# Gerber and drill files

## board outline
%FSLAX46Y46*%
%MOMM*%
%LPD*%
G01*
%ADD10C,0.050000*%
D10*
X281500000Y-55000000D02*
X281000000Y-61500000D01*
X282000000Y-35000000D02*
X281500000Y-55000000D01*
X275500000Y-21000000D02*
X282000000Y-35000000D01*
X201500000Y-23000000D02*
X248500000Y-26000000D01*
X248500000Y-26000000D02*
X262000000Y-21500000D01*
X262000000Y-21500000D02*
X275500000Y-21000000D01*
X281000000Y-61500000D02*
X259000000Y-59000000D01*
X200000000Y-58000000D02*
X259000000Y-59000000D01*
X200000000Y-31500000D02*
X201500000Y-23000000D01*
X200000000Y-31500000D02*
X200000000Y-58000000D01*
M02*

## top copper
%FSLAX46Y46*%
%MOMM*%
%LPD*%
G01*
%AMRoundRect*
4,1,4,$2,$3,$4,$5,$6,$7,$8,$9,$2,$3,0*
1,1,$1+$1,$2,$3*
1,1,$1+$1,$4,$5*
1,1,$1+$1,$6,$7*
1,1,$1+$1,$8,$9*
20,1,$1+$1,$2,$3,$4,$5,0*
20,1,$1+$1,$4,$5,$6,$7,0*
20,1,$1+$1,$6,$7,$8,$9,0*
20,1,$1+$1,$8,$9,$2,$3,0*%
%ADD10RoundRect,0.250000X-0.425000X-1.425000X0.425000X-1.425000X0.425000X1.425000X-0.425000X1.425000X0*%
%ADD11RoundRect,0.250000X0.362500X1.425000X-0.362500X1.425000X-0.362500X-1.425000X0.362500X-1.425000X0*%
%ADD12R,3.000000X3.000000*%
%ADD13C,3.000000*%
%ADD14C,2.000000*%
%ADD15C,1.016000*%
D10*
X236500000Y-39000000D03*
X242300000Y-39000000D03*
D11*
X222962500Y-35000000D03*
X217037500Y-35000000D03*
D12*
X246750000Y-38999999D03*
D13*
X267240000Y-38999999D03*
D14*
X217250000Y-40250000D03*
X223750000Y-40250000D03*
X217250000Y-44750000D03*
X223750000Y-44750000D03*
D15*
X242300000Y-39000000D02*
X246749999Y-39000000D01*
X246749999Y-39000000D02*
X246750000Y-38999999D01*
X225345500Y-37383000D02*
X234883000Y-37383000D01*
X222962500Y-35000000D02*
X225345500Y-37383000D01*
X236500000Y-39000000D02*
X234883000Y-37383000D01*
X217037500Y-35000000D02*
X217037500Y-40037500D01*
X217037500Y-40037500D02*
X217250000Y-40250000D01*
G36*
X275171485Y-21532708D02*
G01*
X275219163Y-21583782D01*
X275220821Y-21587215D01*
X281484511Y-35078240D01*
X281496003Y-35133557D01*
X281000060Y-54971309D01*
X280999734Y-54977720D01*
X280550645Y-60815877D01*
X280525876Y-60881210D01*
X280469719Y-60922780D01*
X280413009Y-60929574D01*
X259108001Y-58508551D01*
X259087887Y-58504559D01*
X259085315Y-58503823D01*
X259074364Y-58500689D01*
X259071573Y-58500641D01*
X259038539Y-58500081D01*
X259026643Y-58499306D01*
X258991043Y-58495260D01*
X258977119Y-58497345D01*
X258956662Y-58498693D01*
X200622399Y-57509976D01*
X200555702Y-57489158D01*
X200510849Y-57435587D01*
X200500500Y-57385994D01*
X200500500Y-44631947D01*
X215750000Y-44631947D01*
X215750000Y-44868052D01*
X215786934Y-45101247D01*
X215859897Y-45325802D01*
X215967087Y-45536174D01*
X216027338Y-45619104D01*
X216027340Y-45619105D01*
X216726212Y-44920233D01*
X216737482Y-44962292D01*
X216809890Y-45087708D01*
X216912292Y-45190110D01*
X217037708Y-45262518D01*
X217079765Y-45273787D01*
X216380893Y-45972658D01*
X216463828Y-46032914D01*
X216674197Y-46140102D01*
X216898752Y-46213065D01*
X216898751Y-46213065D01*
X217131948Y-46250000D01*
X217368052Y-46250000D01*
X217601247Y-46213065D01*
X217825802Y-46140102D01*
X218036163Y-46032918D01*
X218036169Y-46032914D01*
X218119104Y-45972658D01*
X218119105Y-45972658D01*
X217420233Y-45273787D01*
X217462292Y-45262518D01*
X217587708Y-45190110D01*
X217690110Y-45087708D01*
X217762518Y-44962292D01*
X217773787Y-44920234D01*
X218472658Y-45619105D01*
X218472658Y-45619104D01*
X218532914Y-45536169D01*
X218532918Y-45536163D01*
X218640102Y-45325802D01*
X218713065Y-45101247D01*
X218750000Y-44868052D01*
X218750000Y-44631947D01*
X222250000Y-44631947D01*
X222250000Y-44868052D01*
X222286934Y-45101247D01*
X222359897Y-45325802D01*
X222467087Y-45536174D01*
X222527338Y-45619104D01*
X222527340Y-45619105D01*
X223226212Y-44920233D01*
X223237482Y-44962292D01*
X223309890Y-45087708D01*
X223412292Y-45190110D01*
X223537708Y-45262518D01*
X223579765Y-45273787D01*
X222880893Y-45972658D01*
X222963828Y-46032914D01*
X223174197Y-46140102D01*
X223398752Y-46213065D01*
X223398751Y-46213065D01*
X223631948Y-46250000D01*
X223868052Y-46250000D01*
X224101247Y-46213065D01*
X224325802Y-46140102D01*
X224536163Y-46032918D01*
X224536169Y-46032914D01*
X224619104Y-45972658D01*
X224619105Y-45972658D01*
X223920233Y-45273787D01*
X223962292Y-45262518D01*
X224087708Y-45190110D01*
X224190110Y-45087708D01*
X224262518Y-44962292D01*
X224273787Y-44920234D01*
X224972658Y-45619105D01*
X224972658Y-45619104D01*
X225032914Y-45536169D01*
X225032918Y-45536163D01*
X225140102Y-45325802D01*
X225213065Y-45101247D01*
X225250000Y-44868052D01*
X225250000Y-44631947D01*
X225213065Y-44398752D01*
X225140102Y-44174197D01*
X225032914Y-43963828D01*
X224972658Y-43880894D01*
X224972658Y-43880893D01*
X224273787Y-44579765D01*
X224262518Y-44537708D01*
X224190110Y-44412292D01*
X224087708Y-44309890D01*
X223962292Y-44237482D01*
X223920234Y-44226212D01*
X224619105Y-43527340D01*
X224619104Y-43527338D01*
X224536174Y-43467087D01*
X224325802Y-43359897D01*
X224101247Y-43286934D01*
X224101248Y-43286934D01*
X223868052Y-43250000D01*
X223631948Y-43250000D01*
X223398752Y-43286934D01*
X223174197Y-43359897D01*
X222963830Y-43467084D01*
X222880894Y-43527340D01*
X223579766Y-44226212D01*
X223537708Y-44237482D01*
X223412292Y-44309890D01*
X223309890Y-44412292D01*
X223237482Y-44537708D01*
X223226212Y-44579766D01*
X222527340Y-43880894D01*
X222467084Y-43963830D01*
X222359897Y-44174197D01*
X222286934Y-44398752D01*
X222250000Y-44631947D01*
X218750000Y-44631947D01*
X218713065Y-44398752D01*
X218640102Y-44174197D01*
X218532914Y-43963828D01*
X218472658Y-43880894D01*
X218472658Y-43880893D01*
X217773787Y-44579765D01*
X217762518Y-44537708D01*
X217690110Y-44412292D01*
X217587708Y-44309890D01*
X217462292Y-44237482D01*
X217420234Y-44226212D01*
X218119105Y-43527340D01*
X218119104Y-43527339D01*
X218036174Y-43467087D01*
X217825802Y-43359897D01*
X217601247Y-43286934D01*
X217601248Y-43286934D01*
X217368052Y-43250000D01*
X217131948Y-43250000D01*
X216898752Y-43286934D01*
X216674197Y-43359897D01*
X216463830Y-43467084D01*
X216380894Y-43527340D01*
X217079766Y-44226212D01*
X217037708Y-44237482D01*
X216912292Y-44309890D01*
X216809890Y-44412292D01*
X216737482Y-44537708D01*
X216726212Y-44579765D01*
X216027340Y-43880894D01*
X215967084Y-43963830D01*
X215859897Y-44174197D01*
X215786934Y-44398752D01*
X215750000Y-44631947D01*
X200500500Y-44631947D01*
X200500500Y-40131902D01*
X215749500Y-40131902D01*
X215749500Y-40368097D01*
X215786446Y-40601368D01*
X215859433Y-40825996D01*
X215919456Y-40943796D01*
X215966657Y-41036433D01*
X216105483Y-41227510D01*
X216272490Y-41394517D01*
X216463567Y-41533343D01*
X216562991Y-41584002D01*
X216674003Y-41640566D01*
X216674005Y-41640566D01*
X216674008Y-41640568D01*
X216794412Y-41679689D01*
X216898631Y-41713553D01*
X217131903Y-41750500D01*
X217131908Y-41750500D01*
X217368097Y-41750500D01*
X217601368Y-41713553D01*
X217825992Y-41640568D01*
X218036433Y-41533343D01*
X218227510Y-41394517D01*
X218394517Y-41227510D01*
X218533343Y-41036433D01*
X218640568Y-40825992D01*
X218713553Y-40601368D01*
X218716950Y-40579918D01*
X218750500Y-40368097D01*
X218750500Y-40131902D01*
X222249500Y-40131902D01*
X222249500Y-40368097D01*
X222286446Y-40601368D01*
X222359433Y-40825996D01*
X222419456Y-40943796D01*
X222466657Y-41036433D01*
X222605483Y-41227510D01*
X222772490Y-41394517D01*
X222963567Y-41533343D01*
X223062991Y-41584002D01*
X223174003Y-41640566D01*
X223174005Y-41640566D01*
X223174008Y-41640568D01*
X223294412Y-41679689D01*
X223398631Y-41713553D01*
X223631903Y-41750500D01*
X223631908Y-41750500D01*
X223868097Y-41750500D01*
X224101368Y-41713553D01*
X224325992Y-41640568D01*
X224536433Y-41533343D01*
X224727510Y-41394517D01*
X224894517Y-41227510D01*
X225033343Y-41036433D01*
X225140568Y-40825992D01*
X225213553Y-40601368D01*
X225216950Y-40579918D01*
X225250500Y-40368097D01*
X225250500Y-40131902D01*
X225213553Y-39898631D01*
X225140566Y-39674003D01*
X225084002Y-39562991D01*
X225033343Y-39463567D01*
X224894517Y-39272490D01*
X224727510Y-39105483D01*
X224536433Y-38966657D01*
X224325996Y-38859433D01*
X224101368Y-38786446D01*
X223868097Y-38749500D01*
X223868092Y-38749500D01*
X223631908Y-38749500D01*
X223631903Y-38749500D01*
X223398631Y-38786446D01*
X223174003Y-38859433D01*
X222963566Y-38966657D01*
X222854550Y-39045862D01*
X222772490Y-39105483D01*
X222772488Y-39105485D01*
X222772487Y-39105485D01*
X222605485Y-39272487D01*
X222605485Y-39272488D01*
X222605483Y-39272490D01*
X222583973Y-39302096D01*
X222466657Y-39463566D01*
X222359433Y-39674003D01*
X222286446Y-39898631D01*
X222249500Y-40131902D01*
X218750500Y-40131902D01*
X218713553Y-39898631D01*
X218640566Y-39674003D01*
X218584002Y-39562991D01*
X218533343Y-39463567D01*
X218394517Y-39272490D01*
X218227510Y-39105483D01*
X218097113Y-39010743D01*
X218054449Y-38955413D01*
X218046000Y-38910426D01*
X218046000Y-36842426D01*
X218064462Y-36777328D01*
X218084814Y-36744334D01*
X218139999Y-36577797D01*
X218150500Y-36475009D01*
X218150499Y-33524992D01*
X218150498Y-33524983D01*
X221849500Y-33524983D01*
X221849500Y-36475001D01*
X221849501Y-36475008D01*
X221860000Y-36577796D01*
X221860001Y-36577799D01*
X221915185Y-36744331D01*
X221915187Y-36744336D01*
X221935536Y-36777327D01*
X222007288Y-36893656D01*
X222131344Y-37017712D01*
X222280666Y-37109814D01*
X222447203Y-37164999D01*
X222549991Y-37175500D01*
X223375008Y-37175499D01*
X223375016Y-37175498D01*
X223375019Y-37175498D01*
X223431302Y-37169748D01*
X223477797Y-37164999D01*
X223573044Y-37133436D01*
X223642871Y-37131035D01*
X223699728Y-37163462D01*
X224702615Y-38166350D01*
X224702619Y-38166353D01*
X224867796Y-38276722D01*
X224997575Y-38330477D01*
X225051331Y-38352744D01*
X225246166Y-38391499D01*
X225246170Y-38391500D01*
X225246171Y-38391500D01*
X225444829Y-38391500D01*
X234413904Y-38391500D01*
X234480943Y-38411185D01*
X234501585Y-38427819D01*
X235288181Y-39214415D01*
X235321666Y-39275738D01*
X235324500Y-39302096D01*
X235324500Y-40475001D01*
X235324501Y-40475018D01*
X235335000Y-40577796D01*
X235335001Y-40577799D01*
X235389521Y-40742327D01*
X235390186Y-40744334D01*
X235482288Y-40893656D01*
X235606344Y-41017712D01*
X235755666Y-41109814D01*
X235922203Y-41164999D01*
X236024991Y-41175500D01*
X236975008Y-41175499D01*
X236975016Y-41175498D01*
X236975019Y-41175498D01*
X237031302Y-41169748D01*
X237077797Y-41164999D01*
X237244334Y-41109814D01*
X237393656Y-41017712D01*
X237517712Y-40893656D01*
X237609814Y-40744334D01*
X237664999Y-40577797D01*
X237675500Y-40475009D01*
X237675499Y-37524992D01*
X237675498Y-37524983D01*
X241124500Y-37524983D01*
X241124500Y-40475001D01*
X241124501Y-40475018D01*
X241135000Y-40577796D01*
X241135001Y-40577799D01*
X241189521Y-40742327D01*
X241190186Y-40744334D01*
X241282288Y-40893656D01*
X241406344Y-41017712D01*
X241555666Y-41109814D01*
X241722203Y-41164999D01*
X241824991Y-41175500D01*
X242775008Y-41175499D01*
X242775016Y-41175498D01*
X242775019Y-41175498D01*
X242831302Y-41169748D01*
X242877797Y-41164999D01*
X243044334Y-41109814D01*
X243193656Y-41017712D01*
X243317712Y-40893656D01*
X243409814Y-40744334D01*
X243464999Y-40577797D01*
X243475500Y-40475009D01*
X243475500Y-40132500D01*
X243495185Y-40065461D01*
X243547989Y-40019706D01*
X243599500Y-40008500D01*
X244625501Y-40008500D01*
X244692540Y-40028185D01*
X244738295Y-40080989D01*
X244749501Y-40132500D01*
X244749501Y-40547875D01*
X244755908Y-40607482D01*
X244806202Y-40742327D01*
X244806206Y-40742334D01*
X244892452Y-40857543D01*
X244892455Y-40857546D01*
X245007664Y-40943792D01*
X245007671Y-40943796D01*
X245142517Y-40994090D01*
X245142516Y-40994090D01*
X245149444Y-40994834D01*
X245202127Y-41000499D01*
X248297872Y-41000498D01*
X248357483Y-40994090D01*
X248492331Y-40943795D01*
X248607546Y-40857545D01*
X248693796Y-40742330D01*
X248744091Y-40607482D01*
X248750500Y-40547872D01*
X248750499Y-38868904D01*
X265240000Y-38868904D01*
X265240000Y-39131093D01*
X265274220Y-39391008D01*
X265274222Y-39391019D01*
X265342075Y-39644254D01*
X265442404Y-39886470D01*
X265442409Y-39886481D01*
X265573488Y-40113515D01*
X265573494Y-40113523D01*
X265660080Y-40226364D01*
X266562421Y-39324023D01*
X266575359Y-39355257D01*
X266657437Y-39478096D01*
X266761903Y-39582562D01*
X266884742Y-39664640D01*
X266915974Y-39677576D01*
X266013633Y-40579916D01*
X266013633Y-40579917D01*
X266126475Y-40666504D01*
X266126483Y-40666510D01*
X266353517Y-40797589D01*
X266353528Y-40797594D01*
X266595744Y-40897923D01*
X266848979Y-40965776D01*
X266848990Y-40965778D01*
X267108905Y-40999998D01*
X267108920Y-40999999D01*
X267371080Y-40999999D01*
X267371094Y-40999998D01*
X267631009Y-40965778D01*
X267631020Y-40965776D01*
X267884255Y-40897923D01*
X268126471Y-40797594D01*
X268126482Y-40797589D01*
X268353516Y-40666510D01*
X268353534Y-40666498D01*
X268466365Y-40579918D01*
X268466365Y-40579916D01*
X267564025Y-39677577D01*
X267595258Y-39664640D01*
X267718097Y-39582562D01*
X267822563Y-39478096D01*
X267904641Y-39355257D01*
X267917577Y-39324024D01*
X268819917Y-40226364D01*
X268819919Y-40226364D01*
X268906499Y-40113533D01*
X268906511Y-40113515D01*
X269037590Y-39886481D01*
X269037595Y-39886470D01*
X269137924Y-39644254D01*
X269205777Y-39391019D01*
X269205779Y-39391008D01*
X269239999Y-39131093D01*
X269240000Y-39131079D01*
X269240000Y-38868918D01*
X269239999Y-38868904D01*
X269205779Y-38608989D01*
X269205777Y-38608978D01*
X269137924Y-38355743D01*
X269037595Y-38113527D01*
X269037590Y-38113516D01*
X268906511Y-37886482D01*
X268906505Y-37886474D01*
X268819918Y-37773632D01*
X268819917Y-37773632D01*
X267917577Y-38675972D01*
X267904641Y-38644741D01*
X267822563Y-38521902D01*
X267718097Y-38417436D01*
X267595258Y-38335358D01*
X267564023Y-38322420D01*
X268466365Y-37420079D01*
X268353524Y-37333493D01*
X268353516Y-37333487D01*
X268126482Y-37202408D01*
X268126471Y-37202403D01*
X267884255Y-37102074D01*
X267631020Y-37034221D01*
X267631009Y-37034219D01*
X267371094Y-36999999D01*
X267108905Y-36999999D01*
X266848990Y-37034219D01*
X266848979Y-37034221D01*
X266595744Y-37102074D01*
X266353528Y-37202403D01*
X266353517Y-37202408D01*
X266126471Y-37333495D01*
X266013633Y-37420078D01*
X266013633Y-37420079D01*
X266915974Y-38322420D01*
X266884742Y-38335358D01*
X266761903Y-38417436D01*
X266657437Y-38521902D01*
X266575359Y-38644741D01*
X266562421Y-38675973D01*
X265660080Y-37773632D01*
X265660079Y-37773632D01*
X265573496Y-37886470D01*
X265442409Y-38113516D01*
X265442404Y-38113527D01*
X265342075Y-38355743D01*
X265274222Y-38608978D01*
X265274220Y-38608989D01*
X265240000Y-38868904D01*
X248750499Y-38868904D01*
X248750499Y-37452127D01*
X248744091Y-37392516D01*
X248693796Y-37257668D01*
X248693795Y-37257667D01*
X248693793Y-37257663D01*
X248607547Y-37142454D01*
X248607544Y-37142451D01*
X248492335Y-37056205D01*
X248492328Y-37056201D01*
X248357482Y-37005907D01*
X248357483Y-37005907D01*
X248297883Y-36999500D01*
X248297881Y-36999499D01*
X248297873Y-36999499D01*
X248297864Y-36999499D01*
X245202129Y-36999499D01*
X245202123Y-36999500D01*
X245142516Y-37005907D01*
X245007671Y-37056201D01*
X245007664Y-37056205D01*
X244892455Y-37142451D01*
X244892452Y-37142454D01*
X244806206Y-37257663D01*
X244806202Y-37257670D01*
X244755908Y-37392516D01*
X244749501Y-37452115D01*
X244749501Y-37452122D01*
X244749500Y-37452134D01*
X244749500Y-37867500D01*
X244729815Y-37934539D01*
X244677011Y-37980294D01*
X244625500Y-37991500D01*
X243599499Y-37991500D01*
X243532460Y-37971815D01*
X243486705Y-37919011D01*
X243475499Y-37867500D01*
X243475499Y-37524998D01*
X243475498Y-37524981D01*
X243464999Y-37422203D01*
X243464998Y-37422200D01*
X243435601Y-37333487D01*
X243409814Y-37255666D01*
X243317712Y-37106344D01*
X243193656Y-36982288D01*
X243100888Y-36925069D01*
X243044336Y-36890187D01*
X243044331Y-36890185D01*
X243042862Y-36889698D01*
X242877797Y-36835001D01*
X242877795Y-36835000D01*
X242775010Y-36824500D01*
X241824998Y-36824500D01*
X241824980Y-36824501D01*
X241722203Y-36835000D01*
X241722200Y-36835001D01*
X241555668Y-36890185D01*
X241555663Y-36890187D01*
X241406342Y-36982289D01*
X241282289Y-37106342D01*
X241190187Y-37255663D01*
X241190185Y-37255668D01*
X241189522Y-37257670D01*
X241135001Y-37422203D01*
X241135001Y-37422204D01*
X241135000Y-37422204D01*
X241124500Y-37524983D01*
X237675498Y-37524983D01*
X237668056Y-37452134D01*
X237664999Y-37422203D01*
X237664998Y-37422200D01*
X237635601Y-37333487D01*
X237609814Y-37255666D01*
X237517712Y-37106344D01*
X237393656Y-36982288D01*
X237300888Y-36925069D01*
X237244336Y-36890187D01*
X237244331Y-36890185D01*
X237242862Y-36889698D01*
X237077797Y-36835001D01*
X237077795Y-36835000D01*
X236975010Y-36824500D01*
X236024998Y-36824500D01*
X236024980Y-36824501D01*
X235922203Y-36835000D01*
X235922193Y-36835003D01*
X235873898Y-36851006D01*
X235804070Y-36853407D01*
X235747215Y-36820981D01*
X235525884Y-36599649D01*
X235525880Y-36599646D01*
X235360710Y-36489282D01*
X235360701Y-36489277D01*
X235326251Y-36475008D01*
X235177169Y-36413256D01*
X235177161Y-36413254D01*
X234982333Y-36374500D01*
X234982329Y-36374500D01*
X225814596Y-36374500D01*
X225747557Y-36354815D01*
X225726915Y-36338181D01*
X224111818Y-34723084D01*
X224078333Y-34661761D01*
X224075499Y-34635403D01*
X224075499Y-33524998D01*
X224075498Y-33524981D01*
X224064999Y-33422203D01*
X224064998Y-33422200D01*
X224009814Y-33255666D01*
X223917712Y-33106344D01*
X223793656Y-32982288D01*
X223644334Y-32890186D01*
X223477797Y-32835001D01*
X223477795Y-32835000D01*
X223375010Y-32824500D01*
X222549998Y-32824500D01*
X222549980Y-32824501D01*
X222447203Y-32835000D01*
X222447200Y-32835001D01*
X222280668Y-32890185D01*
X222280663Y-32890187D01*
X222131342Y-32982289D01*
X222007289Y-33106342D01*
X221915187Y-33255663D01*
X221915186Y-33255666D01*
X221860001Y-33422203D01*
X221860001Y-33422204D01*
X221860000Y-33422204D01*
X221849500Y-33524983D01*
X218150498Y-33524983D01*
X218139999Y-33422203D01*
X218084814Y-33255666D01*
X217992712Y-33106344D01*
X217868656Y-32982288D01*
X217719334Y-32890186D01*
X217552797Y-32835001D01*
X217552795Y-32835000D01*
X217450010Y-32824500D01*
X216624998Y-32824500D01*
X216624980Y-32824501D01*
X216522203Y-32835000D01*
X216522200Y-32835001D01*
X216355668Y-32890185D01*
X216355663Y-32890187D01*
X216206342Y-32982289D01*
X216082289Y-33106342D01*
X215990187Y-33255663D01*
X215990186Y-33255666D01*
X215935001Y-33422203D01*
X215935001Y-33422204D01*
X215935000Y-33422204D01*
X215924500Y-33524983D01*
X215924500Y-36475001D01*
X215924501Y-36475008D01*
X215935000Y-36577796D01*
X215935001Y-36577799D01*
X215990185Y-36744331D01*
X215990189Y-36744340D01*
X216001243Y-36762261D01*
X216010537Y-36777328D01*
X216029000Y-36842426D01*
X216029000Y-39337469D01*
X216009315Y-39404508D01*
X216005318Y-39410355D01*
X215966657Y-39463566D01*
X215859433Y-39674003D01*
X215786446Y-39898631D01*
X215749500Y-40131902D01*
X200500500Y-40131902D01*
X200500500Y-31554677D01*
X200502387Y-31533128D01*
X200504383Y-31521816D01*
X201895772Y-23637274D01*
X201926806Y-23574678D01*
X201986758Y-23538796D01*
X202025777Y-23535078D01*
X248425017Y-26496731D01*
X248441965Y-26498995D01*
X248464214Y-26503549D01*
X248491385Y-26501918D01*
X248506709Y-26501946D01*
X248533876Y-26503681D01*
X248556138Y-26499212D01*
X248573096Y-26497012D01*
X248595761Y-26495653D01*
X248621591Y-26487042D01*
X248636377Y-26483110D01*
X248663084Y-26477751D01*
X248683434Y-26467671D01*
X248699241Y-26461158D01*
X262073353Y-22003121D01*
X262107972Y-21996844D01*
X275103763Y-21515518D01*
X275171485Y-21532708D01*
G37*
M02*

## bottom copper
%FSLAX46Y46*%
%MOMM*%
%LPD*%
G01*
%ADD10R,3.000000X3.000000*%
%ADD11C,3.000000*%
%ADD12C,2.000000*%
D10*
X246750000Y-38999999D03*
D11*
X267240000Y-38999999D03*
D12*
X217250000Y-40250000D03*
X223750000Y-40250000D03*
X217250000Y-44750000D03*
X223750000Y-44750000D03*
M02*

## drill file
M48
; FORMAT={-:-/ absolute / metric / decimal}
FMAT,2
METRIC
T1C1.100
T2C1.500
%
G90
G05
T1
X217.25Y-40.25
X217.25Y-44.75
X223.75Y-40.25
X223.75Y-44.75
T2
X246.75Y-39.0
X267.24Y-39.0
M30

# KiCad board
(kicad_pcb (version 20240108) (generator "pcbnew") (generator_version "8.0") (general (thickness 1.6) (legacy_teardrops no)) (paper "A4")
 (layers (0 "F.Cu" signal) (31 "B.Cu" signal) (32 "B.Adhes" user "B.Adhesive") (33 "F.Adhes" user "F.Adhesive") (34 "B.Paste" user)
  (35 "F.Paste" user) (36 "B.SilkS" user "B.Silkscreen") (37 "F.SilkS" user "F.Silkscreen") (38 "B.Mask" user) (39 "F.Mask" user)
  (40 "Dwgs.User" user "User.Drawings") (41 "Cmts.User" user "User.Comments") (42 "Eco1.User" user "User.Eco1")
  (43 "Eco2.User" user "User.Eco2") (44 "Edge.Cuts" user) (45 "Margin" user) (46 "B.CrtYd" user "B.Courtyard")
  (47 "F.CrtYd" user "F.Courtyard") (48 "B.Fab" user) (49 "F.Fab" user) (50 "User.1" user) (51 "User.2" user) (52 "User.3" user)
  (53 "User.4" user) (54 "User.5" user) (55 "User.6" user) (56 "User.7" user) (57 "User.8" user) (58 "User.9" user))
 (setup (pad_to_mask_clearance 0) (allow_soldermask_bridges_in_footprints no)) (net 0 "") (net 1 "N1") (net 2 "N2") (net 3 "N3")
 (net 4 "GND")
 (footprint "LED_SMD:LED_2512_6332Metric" (layer "F.Cu") (at 239.4 39)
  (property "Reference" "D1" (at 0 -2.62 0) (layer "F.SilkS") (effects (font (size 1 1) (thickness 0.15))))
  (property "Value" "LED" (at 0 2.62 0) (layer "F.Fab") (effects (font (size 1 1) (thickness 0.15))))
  (pad "1" smd roundrect (at -2.9 0) (size 1.35 3.35) (layers "F.Cu" "F.Paste" "F.Mask") (roundrect_rratio 0.185185) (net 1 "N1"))
  (pad "2" smd roundrect (at 2.9 0) (size 1.35 3.35) (layers "F.Cu" "F.Paste" "F.Mask") (roundrect_rratio 0.185185) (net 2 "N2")))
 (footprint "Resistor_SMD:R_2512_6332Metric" (layer "F.Cu") (at 220 35 180)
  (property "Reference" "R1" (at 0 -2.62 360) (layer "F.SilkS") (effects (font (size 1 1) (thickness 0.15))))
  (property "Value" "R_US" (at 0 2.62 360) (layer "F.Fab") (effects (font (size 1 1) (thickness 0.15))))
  (pad "1" smd roundrect (at -2.9625 0 180) (size 1.225 3.35) (layers "F.Cu" "F.Paste" "F.Mask") (roundrect_rratio 0.204082) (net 1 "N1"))
  (pad "2" smd roundrect (at 2.9625 0 180) (size 1.225 3.35) (layers "F.Cu" "F.Paste" "F.Mask") (roundrect_rratio 0.204082) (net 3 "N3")))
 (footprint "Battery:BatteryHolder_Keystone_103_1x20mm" (layer "F.Cu") (at 246.75 38.999999)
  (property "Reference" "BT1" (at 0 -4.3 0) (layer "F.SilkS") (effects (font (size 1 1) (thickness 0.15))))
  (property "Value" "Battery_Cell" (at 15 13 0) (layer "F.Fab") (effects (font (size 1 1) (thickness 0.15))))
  (pad "1" thru_hole rect (at 0 0) (size 3 3) (drill 1.5) (layers "*.Cu" "*.Mask") (remove_unused_layers no) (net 2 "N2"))
  (pad "2" thru_hole circle (at 20.49 0) (size 3 3) (drill 1.5) (layers "*.Cu" "*.Mask") (remove_unused_layers no) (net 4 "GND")))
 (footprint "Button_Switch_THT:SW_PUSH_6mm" (layer "F.Cu") (at 217.25 40.25)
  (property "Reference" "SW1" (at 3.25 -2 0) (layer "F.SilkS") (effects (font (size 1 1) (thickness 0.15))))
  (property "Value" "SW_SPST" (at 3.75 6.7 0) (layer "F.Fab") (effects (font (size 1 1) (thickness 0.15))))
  (pad "1" thru_hole circle (at 0 0 90) (size 2 2) (drill 1.1) (layers "*.Cu" "*.Mask") (remove_unused_layers no) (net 3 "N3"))
  (pad "1" thru_hole circle (at 6.5 0 90) (size 2 2) (drill 1.1) (layers "*.Cu" "*.Mask") (remove_unused_layers no) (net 3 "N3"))
  (pad "2" thru_hole circle (at 0 4.5 90) (size 2 2) (drill 1.1) (layers "*.Cu" "*.Mask") (remove_unused_layers no) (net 4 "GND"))
  (pad "2" thru_hole circle (at 6.5 4.5 90) (size 2 2) (drill 1.1) (layers "*.Cu" "*.Mask") (remove_unused_layers no) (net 4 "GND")))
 (gr_line (start 281.5 55) (end 281 61.5) (stroke (width 0.05) (type default)) (layer "Edge.Cuts"))
 (gr_line (start 282 35) (end 281.5 55) (stroke (width 0.05) (type default)) (layer "Edge.Cuts"))
 (gr_line (start 275.5 21) (end 282 35) (stroke (width 0.05) (type default)) (layer "Edge.Cuts"))
 (gr_line (start 201.5 23) (end 248.5 26) (stroke (width 0.05) (type default)) (layer "Edge.Cuts"))
 (gr_line (start 248.5 26) (end 262 21.5) (stroke (width 0.05) (type default)) (layer "Edge.Cuts"))
 (gr_line (start 262 21.5) (end 275.5 21) (stroke (width 0.05) (type default)) (layer "Edge.Cuts"))
 (gr_line (start 281 61.5) (end 259 59) (stroke (width 0.05) (type default)) (layer "Edge.Cuts"))
 (gr_line (start 200 58) (end 259 59) (stroke (width 0.05) (type default)) (layer "Edge.Cuts"))
 (gr_line (start 200 31.5) (end 201.5 23) (stroke (width 0.05) (type default)) (layer "Edge.Cuts"))
 (gr_line (start 200 31.5) (end 200 58) (stroke (width 0.05) (type default)) (layer "Edge.Cuts"))
 (segment (start 242.3 39) (end 246.749999 39) (width 1.016) (layer "F.Cu") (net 2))
 (segment (start 246.749999 39) (end 246.75 38.999999) (width 1.016) (layer "F.Cu") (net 2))
 (segment (start 225.3455 37.383) (end 234.883 37.383) (width 1.016) (layer "F.Cu") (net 1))
 (segment (start 222.9625 35) (end 225.3455 37.383) (width 1.016) (layer "F.Cu") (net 1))
 (segment (start 236.5 39) (end 234.883 37.383) (width 1.016) (layer "F.Cu") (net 1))
 (segment (start 217.0375 35) (end 217.0375 40.0375) (width 1.016) (layer "F.Cu") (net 3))
 (segment (start 217.0375 40.0375) (end 217.25 40.25) (width 1.016) (layer "F.Cu") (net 3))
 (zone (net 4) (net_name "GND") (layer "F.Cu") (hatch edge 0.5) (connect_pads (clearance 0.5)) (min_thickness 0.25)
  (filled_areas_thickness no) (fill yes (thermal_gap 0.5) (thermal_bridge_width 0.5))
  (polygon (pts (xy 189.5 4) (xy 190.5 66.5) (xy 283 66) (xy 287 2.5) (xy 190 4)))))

